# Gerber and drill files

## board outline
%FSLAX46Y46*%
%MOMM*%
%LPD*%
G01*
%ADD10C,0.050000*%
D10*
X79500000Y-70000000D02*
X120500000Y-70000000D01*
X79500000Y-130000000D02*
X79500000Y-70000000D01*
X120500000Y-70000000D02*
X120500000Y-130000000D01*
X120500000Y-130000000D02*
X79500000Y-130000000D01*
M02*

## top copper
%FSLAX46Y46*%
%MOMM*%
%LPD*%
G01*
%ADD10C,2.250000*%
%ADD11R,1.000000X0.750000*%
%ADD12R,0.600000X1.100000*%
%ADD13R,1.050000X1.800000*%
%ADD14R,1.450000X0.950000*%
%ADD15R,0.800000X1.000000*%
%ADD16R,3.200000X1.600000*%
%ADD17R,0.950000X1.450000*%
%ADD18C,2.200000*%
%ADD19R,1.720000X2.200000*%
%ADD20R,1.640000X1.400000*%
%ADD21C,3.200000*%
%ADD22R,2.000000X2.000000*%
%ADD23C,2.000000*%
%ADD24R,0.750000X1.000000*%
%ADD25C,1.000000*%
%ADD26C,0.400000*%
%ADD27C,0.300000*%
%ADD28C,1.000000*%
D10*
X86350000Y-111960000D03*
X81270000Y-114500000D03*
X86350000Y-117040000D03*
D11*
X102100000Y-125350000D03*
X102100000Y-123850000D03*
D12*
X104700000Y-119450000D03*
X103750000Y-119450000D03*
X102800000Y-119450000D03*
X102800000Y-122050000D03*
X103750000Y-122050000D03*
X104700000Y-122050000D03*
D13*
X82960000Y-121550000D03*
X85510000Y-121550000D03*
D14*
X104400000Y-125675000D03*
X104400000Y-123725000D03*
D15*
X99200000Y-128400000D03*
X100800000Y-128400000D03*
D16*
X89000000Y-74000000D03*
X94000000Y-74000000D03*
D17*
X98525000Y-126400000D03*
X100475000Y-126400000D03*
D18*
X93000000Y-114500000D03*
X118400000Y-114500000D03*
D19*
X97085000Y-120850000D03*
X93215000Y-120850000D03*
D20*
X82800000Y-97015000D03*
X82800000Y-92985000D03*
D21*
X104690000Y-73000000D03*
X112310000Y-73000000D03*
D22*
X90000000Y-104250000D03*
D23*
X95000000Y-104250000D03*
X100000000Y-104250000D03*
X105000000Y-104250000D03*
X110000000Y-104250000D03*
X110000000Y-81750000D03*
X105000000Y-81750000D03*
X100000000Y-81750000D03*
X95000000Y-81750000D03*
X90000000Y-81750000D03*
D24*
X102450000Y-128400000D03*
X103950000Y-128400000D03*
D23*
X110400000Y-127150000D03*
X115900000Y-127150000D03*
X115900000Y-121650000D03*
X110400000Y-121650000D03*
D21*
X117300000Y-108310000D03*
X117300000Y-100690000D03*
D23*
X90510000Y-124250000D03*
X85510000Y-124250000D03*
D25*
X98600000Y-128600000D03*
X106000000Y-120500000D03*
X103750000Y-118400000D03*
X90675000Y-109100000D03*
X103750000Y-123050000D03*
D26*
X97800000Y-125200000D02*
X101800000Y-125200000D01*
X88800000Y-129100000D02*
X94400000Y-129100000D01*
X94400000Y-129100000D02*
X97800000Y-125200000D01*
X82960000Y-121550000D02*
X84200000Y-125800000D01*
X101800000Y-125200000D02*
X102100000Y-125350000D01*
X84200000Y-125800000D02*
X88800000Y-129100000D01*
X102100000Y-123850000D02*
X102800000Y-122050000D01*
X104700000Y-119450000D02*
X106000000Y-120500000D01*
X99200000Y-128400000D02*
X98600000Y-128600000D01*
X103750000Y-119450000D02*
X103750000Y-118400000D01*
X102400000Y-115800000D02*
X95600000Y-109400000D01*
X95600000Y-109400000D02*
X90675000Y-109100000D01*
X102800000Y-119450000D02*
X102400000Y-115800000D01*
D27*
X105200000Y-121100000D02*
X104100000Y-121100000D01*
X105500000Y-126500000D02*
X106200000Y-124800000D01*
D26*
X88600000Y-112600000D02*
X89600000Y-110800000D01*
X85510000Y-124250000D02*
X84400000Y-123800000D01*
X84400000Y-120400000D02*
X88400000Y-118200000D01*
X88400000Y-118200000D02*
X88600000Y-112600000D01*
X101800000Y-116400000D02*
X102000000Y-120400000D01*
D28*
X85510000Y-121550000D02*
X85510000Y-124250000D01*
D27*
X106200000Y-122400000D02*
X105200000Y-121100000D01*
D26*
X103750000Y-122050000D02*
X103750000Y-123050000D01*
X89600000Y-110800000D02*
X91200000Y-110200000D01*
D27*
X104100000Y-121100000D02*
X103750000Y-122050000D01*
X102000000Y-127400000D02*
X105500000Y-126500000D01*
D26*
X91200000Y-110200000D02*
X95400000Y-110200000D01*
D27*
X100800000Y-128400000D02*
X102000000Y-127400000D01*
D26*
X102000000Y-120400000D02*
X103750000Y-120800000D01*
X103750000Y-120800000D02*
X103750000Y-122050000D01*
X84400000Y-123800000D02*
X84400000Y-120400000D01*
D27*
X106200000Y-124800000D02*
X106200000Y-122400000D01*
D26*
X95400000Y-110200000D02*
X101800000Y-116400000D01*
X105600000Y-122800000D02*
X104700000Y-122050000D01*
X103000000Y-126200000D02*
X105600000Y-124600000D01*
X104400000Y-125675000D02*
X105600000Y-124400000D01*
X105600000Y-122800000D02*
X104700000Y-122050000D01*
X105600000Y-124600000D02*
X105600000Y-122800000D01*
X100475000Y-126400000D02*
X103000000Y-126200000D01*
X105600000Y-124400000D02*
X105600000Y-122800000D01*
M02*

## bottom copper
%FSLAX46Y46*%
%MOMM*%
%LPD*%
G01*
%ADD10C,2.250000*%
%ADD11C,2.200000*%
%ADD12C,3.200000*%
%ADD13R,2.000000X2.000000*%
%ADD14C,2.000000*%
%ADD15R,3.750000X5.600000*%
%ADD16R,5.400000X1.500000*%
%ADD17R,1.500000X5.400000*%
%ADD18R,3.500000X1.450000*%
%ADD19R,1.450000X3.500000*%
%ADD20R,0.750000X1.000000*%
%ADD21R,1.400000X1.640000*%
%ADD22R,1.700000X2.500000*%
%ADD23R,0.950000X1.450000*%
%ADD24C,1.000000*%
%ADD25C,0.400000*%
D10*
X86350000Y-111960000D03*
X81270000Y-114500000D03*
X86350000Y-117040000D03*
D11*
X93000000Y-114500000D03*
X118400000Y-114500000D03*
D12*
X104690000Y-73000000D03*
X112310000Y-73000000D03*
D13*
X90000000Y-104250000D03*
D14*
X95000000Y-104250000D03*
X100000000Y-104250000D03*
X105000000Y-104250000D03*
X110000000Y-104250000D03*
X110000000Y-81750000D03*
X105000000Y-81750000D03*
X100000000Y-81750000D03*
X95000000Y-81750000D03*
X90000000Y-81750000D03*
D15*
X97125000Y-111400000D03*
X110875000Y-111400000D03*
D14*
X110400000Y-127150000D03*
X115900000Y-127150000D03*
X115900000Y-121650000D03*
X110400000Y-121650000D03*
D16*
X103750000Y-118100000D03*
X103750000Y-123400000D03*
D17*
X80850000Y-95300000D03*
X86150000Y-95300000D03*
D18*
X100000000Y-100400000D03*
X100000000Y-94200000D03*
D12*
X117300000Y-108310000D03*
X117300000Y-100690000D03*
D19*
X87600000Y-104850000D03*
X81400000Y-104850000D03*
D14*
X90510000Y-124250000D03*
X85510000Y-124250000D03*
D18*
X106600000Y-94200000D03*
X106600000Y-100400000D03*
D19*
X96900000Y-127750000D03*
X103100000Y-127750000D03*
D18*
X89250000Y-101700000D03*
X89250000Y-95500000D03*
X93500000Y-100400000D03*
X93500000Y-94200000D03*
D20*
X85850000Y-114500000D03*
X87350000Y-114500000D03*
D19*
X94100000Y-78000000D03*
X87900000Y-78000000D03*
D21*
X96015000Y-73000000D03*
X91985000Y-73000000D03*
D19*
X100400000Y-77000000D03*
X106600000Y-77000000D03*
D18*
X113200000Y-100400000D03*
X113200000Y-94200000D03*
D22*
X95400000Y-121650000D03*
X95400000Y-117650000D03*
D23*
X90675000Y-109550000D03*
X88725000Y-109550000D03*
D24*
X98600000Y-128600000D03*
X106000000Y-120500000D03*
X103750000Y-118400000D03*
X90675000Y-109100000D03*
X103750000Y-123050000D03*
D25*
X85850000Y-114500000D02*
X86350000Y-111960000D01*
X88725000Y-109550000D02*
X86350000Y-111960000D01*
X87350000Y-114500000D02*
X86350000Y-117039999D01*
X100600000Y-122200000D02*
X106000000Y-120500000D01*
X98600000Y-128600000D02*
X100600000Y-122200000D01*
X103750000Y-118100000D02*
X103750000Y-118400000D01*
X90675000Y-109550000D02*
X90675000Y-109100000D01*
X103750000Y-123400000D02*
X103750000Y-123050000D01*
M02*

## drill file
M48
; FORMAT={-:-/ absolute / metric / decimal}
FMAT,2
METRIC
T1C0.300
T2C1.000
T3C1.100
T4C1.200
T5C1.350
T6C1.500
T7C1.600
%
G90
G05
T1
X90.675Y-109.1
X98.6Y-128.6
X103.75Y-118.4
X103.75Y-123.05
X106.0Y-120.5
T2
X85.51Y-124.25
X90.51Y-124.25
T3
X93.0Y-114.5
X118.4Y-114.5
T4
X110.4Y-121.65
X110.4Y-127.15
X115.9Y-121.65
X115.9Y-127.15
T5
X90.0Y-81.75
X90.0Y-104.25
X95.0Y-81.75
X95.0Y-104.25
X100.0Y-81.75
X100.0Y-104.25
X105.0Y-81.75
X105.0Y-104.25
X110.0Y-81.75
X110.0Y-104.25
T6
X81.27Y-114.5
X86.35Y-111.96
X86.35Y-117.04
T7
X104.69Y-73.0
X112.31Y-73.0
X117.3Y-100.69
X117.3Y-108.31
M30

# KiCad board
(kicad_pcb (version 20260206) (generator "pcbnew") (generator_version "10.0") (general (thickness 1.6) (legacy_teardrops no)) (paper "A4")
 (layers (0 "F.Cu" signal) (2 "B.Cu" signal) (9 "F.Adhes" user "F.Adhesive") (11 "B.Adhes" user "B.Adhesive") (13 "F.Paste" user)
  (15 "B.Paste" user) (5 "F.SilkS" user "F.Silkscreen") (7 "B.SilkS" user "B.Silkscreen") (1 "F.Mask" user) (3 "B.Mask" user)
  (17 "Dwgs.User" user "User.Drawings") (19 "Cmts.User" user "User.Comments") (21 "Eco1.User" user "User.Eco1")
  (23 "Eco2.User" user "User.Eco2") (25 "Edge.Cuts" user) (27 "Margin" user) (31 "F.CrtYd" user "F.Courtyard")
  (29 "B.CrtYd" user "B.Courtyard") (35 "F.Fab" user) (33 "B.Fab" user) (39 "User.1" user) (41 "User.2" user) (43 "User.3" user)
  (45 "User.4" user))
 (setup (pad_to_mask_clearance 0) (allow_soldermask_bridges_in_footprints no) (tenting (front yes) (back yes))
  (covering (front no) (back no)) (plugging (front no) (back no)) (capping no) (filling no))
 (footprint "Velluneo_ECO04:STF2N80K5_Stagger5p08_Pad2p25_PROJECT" (layer "F.Cu") (at 86.35 114.5 -90)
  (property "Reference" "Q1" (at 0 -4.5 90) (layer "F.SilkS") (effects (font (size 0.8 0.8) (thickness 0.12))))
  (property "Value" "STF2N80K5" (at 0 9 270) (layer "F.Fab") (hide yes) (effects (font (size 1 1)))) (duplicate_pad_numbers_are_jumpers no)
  (pad "1" thru_hole circle (at -2.54 0 270) (size 2.25 2.25) (drill 1.5) (layers "*.Cu" "*.Mask") (remove_unused_layers no) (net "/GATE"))
  (pad "2" thru_hole circle (at 0 5.08 270) (size 2.25 2.25) (drill 1.5) (layers "*.Cu" "*.Mask") (remove_unused_layers no) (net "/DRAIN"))
  (pad "3" thru_hole circle (at 2.54 0 270) (size 2.25 2.25) (drill 1.5) (layers "*.Cu" "*.Mask") (remove_unused_layers no) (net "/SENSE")))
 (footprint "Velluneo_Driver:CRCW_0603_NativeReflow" (layer "F.Cu") (at 102.1 124.6 90)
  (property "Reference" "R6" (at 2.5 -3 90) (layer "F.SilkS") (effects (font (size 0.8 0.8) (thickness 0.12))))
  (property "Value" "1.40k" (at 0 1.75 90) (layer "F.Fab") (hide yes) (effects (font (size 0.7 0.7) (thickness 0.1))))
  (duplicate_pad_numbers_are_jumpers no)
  (pad "1" smd rect (at -0.75 0 90) (size 0.75 1) (layers "F.Cu" "F.Mask" "F.Paste") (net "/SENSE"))
  (pad "2" smd rect (at 0.75 0 90) (size 0.75 1) (layers "F.Cu" "F.Mask" "F.Paste") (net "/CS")))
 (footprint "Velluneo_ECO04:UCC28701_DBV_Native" (layer "F.Cu") (at 103.75 120.75 -90)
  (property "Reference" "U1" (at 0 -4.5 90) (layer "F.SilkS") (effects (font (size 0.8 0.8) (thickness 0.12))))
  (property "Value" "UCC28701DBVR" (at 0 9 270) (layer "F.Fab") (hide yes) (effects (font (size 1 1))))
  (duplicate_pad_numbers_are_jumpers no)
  (pad "1" smd rect (at -1.3 -0.95 270) (size 1.1 0.6) (layers "F.Cu" "F.Mask" "F.Paste") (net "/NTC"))
  (pad "2" smd rect (at -1.3 0 270) (size 1.1 0.6) (layers "F.Cu" "F.Mask" "F.Paste") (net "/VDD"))
  (pad "3" smd rect (at -1.3 0.95 270) (size 1.1 0.6) (layers "F.Cu" "F.Mask" "F.Paste") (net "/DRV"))
  (pad "4" smd rect (at 1.3 0.95 270) (size 1.1 0.6) (layers "F.Cu" "F.Mask" "F.Paste") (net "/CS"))
  (pad "5" smd rect (at 1.3 0 270) (size 1.1 0.6) (layers "F.Cu" "F.Mask" "F.Paste") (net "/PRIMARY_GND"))
  (pad "6" smd rect (at 1.3 -0.95 270) (size 1.1 0.6) (layers "F.Cu" "F.Mask" "F.Paste") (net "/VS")))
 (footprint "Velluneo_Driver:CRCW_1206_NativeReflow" (layer "F.Cu") (at 84.235 121.55)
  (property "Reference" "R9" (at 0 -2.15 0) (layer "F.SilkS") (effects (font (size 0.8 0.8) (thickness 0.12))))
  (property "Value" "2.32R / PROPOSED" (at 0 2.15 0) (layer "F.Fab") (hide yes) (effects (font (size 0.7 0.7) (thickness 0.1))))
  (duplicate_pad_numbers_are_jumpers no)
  (pad "1" smd rect (at -1.275 0) (size 1.05 1.8) (layers "F.Cu" "F.Mask" "F.Paste") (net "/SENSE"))
  (pad "2" smd rect (at 1.275 0) (size 1.05 1.8) (layers "F.Cu" "F.Mask" "F.Paste") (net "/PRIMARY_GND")))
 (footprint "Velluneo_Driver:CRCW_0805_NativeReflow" (layer "F.Cu") (at 104.4 124.7 90)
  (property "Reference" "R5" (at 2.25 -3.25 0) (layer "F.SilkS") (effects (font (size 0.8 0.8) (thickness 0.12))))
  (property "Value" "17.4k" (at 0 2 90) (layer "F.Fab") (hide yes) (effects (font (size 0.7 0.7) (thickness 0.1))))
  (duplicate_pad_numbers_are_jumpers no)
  (pad "1" smd rect (at -0.975 0 90) (size 0.95 1.45) (layers "F.Cu" "F.Mask" "F.Paste") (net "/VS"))
  (pad "2" smd rect (at 0.975 0 90) (size 0.95 1.45) (layers "F.Cu" "F.Mask" "F.Paste") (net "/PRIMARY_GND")))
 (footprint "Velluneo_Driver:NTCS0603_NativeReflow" (layer "F.Cu") (at 100 128.4)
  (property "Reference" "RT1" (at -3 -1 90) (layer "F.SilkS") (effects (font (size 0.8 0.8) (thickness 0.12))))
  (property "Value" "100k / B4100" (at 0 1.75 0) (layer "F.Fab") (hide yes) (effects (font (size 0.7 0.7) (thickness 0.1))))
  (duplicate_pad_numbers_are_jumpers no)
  (pad "1" smd rect (at -0.8 0) (size 0.8 1) (layers "F.Cu" "F.Mask" "F.Paste") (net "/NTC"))
  (pad "2" smd rect (at 0.8 0) (size 0.8 1) (layers "F.Cu" "F.Mask" "F.Paste") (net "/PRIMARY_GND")))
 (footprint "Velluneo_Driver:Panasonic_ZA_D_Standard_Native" (layer "F.Cu") (at 91.5 74)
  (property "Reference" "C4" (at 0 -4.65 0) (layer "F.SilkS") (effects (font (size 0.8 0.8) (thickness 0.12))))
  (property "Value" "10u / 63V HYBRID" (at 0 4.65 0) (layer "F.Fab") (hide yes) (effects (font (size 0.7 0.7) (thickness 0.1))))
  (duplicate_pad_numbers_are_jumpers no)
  (pad "1" smd rect (at -2.5 0) (size 3.2 1.6) (layers "F.Cu" "F.Mask" "F.Paste") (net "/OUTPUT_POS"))
  (pad "2" smd rect (at 2.5 0) (size 3.2 1.6) (layers "F.Cu" "F.Mask" "F.Paste") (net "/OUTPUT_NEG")))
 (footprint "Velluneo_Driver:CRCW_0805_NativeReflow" (layer "F.Cu") (at 99.5 126.4)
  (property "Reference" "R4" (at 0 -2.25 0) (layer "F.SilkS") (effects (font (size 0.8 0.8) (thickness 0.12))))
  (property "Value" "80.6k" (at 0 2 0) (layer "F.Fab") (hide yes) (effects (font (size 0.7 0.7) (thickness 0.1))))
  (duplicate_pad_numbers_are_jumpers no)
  (pad "1" smd rect (at -0.975 0) (size 0.95 1.45) (layers "F.Cu" "F.Mask" "F.Paste") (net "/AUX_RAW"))
  (pad "2" smd rect (at 0.975 0) (size 0.95 1.45) (layers "F.Cu" "F.Mask" "F.Paste") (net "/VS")))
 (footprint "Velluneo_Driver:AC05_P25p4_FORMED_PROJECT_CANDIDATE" (layer "F.Cu") (at 105.7 114.5)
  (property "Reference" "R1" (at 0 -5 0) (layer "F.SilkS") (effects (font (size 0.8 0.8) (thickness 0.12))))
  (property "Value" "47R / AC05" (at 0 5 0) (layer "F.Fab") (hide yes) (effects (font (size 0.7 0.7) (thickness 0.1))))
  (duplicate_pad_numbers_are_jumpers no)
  (pad "1" thru_hole circle (at -12.7 0) (size 2.2 2.2) (drill 1.1) (layers "*.Cu" "*.Mask") (remove_unused_layers no) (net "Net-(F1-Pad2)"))
  (pad "2" thru_hole circle (at 12.7 0) (size 2.2 2.2) (drill 1.1) (layers "*.Cu" "*.Mask") (remove_unused_layers no)
   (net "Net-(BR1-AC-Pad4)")))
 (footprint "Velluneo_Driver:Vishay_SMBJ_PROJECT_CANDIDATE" (layer "F.Cu") (at 95.15 120.85 180)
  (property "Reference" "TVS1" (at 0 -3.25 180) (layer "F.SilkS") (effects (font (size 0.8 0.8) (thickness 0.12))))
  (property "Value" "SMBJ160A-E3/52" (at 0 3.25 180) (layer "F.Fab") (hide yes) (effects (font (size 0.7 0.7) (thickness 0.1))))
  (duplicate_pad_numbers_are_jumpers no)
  (pad "1" smd rect (at -1.935 0 180) (size 1.72 2.2) (layers "F.Cu" "F.Mask" "F.Paste") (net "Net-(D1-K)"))
  (pad "2" smd rect (at 1.935 0 180) (size 1.72 2.2) (layers "F.Cu" "F.Mask" "F.Paste") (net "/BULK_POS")))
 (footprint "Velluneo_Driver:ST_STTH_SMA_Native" (layer "F.Cu") (at 82.8 95 90)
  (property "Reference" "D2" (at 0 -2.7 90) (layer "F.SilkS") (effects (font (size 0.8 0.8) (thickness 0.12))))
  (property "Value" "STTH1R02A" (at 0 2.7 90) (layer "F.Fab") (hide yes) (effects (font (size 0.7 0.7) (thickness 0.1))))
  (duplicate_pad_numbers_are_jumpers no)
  (pad "1" smd rect (at -2.015 0 90) (size 1.4 1.64) (layers "F.Cu" "F.Mask" "F.Paste") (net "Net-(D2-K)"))
  (pad "2" smd rect (at 2.015 0 90) (size 1.4 1.64) (layers "F.Cu" "F.Mask" "F.Paste") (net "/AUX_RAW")))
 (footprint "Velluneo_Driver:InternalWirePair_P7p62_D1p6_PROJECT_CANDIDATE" (layer "F.Cu") (at 108.5 73)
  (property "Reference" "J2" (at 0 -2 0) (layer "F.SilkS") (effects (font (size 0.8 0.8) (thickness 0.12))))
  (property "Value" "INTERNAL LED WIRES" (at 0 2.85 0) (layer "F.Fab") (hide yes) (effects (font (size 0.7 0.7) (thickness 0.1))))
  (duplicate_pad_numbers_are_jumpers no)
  (pad "1" thru_hole circle (at -3.81 0) (size 3.2 3.2) (drill 1.6) (layers "*.Cu" "*.Mask") (remove_unused_layers no) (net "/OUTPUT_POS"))
  (pad "2" thru_hole circle (at 3.81 0) (size 3.2 3.2) (drill 1.6) (layers "*.Cu" "*.Mask") (remove_unused_layers no) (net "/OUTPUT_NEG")))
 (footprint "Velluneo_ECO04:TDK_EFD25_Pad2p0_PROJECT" (layer "F.Cu") (at 100 93)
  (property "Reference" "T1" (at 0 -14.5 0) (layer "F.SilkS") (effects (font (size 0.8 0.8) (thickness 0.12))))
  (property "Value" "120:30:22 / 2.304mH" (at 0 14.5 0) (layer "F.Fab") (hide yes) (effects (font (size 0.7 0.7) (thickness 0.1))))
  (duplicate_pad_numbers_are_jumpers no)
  (pad "1" thru_hole rect (at -10 11.25) (size 2 2) (drill 1.35) (layers "*.Cu" "*.Mask") (remove_unused_layers no) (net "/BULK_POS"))
  (pad "2" thru_hole circle (at -5 11.25) (size 2 2) (drill 1.35) (layers "*.Cu" "*.Mask") (remove_unused_layers no) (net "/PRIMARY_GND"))
  (pad "3" thru_hole circle (at 0 11.25) (size 2 2) (drill 1.35) (layers "*.Cu" "*.Mask") (remove_unused_layers no)
   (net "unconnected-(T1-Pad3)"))
  (pad "4" thru_hole circle (at 5 11.25) (size 2 2) (drill 1.35) (layers "*.Cu" "*.Mask") (remove_unused_layers no) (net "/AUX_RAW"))
  (pad "5" thru_hole circle (at 10 11.25) (size 2 2) (drill 1.35) (layers "*.Cu" "*.Mask") (remove_unused_layers no) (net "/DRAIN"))
  (pad "6" thru_hole circle (at 10 -11.25) (size 2 2) (drill 1.35) (layers "*.Cu" "*.Mask") (remove_unused_layers no) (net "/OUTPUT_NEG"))
  (pad "7" thru_hole circle (at 5 -11.25) (size 2 2) (drill 1.35) (layers "*.Cu" "*.Mask") (remove_unused_layers no)
   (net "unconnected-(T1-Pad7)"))
  (pad "8" thru_hole circle (at 0 -11.25) (size 2 2) (drill 1.35) (layers "*.Cu" "*.Mask") (remove_unused_layers no)
   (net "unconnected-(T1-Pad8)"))
  (pad "9" thru_hole circle (at -5 -11.25) (size 2 2) (drill 1.35) (layers "*.Cu" "*.Mask") (remove_unused_layers no)
   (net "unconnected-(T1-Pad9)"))
  (pad "10" thru_hole circle (at -10 -11.25) (size 2 2) (drill 1.35) (layers "*.Cu" "*.Mask") (remove_unused_layers no)
   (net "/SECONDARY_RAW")))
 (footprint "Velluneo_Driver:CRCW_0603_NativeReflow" (layer "F.Cu") (at 103.2 128.4)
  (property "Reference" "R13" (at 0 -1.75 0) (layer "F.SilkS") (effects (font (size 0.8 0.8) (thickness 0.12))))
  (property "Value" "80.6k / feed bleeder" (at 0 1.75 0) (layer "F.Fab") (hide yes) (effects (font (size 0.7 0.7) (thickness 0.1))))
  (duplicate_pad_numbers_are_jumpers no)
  (pad "1" smd rect (at -0.75 0) (size 0.75 1) (layers "F.Cu" "F.Mask" "F.Paste") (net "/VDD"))
  (pad "2" smd rect (at 0.75 0) (size 0.75 1) (layers "F.Cu" "F.Mask" "F.Paste") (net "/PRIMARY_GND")))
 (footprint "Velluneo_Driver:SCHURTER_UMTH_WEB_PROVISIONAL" (layer "B.Cu") (at 104 111.4)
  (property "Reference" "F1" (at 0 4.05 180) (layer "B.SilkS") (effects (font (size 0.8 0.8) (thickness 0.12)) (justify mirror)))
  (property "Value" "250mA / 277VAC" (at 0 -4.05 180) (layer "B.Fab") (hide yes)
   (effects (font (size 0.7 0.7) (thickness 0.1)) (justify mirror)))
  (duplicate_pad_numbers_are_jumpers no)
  (pad "1" smd rect (at -6.875 0) (size 3.75 5.6) (layers "B.Cu" "B.Mask" "B.Paste") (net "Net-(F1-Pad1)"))
  (pad "2" smd rect (at 6.875 0) (size 3.75 5.6) (layers "B.Cu" "B.Mask" "B.Paste") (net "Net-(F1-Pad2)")))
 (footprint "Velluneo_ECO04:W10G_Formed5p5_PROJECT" (layer "B.Cu") (at 113.15 124.4)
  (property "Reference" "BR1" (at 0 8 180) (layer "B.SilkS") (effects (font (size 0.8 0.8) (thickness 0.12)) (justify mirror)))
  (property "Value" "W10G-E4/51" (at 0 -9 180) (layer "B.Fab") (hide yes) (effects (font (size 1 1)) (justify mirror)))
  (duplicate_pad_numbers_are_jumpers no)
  (pad "1" thru_hole circle (at -2.75 2.75) (size 2 2) (drill 1.2) (layers "*.Cu" "*.Mask") (remove_unused_layers no) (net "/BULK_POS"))
  (pad "2" thru_hole circle (at 2.75 2.75) (size 2 2) (drill 1.2) (layers "*.Cu" "*.Mask") (remove_unused_layers no)
   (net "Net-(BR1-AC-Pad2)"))
  (pad "3" thru_hole circle (at 2.75 -2.75) (size 2 2) (drill 1.2) (layers "*.Cu" "*.Mask") (remove_unused_layers no) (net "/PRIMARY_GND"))
  (pad "4" thru_hole circle (at -2.75 -2.75) (size 2 2) (drill 1.2) (layers "*.Cu" "*.Mask") (remove_unused_layers no)
   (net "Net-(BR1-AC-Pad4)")))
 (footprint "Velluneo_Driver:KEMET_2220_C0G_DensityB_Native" (layer "B.Cu") (at 103.75 120.75 -90)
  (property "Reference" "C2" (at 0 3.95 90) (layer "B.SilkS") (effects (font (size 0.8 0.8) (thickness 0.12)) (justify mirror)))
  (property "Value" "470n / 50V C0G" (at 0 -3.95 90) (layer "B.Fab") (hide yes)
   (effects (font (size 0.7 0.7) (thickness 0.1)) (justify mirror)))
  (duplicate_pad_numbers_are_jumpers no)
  (pad "1" smd rect (at -2.65 0 270) (size 1.5 5.4) (layers "B.Cu" "B.Mask" "B.Paste") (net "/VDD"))
  (pad "2" smd rect (at 2.65 0 270) (size 1.5 5.4) (layers "B.Cu" "B.Mask" "B.Paste") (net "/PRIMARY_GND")))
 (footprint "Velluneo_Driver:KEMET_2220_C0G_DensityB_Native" (layer "B.Cu") (at 83.5 95.3)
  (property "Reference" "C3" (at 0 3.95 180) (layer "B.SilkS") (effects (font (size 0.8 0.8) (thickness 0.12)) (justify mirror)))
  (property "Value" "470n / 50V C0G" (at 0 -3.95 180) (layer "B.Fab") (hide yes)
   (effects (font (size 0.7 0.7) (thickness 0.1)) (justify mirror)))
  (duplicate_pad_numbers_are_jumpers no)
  (pad "1" smd rect (at -2.65 0) (size 1.5 5.4) (layers "B.Cu" "B.Mask" "B.Paste") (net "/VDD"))
  (pad "2" smd rect (at 2.65 0) (size 1.5 5.4) (layers "B.Cu" "B.Mask" "B.Paste") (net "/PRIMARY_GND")))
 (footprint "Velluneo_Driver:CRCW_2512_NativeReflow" (layer "B.Cu") (at 100 97.3 90)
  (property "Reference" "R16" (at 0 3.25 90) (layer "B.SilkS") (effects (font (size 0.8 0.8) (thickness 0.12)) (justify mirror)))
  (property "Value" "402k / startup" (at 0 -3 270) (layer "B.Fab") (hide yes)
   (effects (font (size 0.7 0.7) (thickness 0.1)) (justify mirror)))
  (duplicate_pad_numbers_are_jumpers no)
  (pad "1" smd rect (at -3.1 0 90) (size 1.45 3.5) (layers "B.Cu" "B.Mask" "B.Paste") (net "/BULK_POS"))
  (pad "2" smd rect (at 3.1 0 90) (size 1.45 3.5) (layers "B.Cu" "B.Mask" "B.Paste") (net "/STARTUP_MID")))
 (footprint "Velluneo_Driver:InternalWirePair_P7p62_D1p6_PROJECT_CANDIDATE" (layer "B.Cu") (at 117.3 104.5 90)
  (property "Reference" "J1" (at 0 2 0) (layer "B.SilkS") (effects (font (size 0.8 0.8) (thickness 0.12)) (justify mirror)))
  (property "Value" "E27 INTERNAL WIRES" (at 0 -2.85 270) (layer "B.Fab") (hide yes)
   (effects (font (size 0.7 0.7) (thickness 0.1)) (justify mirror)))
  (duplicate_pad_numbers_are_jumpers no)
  (pad "1" thru_hole circle (at -3.81 0 90) (size 3.2 3.2) (drill 1.6) (layers "*.Cu" "*.Mask") (remove_unused_layers no)
   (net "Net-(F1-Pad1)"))
  (pad "2" thru_hole circle (at 3.81 0 90) (size 3.2 3.2) (drill 1.6) (layers "*.Cu" "*.Mask") (remove_unused_layers no)
   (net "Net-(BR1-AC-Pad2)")))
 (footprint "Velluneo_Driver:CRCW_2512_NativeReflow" (layer "B.Cu") (at 84.5 104.85 180)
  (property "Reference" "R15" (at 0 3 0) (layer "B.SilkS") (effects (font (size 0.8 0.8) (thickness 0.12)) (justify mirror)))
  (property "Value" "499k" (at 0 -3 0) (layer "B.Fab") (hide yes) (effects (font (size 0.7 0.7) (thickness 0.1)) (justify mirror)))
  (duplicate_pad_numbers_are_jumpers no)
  (pad "1" smd rect (at -3.1 0 180) (size 1.45 3.5) (layers "B.Cu" "B.Mask" "B.Paste") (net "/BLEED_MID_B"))
  (pad "2" smd rect (at 3.1 0 180) (size 1.45 3.5) (layers "B.Cu" "B.Mask" "B.Paste") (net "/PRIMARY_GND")))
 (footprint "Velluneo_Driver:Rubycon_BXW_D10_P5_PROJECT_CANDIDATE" (layer "B.Cu") (at 88.01 124.25 180)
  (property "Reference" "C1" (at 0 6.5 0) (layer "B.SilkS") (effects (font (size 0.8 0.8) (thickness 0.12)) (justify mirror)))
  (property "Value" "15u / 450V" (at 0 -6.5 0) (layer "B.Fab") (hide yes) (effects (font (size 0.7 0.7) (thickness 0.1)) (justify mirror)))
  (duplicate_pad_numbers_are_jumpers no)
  (pad "1" thru_hole circle (at -2.5 0 180) (size 2 2) (drill 1) (layers "*.Cu" "*.Mask") (remove_unused_layers no) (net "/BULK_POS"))
  (pad "2" thru_hole circle (at 2.5 0 180) (size 2 2) (drill 1) (layers "*.Cu" "*.Mask") (remove_unused_layers no) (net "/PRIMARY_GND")))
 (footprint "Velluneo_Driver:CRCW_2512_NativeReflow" (layer "B.Cu") (at 106.6 97.3 -90)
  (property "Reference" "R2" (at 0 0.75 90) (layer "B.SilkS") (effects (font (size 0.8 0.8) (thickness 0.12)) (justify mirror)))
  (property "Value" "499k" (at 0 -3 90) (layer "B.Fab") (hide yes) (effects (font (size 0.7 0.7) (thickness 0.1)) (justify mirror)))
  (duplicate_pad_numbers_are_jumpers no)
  (pad "1" smd rect (at -3.1 0 270) (size 1.45 3.5) (layers "B.Cu" "B.Mask" "B.Paste") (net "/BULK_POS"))
  (pad "2" smd rect (at 3.1 0 270) (size 1.45 3.5) (layers "B.Cu" "B.Mask" "B.Paste") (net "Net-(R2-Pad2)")))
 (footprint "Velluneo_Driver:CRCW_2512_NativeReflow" (layer "B.Cu") (at 100 127.75)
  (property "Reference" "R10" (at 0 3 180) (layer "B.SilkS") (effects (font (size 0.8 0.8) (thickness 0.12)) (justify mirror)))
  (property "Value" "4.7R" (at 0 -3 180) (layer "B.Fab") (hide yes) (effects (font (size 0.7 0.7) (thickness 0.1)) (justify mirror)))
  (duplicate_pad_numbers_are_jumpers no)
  (pad "1" smd rect (at -3.1 0) (size 1.45 3.5) (layers "B.Cu" "B.Mask" "B.Paste") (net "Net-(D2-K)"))
  (pad "2" smd rect (at 3.1 0) (size 1.45 3.5) (layers "B.Cu" "B.Mask" "B.Paste") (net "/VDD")))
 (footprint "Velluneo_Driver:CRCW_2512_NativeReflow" (layer "B.Cu") (at 89.25 98.6 90)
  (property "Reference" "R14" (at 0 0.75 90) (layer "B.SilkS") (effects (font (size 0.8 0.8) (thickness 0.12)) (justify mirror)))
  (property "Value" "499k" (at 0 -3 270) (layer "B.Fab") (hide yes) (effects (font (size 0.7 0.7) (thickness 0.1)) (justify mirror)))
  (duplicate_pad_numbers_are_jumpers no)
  (pad "1" smd rect (at -3.1 0 90) (size 1.45 3.5) (layers "B.Cu" "B.Mask" "B.Paste") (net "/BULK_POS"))
  (pad "2" smd rect (at 3.1 0 90) (size 1.45 3.5) (layers "B.Cu" "B.Mask" "B.Paste") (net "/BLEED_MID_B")))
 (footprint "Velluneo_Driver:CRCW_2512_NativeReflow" (layer "B.Cu") (at 93.5 97.3 90)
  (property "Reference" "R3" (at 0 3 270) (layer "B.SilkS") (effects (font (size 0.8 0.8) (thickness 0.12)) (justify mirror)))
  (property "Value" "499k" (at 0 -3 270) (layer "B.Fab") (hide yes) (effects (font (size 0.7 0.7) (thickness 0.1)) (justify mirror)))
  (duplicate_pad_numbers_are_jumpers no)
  (pad "1" smd rect (at -3.1 0 90) (size 1.45 3.5) (layers "B.Cu" "B.Mask" "B.Paste") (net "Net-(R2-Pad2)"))
  (pad "2" smd rect (at 3.1 0 90) (size 1.45 3.5) (layers "B.Cu" "B.Mask" "B.Paste") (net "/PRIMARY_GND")))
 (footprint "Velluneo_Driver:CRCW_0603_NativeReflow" (layer "B.Cu") (at 86.6 114.5)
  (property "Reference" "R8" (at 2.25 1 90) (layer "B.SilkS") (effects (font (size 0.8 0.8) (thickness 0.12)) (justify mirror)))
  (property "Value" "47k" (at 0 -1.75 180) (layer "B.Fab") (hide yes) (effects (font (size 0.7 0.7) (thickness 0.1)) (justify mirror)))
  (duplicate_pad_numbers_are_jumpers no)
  (pad "1" smd rect (at -0.75 0) (size 0.75 1) (layers "B.Cu" "B.Mask" "B.Paste") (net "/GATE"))
  (pad "2" smd rect (at 0.75 0) (size 0.75 1) (layers "B.Cu" "B.Mask" "B.Paste") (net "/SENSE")))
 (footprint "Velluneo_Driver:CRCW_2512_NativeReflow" (layer "B.Cu") (at 91 78 180)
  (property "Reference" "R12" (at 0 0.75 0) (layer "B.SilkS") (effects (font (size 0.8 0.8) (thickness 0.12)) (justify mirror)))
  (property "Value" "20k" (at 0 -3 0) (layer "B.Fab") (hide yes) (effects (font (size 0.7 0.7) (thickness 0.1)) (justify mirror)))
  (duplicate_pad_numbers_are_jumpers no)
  (pad "1" smd rect (at -3.1 0 180) (size 1.45 3.5) (layers "B.Cu" "B.Mask" "B.Paste") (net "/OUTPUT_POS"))
  (pad "2" smd rect (at 3.1 0 180) (size 1.45 3.5) (layers "B.Cu" "B.Mask" "B.Paste") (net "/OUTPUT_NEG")))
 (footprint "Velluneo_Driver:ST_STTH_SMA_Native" (layer "B.Cu") (at 94 73 180)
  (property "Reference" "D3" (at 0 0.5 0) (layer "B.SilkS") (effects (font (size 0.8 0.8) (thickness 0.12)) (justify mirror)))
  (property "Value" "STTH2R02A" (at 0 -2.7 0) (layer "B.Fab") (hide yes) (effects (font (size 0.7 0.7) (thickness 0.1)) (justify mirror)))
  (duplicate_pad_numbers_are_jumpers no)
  (pad "1" smd rect (at -2.015 0 180) (size 1.4 1.64) (layers "B.Cu" "B.Mask" "B.Paste") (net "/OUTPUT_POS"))
  (pad "2" smd rect (at 2.015 0 180) (size 1.4 1.64) (layers "B.Cu" "B.Mask" "B.Paste") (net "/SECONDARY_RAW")))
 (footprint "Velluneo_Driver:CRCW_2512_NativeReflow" (layer "B.Cu") (at 103.5 77)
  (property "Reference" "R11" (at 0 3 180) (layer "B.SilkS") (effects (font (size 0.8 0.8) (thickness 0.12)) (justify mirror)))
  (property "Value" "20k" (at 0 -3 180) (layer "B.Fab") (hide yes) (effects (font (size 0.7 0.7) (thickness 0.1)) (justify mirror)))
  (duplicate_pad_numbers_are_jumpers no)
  (pad "1" smd rect (at -3.1 0) (size 1.45 3.5) (layers "B.Cu" "B.Mask" "B.Paste") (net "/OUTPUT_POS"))
  (pad "2" smd rect (at 3.1 0) (size 1.45 3.5) (layers "B.Cu" "B.Mask" "B.Paste") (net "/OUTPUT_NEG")))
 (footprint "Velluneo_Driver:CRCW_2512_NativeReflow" (layer "B.Cu") (at 113.2 97.3 90)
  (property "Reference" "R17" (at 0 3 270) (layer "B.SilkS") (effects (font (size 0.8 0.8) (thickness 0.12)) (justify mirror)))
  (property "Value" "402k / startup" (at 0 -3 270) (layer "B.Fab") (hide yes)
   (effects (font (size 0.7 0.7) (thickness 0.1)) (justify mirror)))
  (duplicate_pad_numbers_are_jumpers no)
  (pad "1" smd rect (at -3.1 0 90) (size 1.45 3.5) (layers "B.Cu" "B.Mask" "B.Paste") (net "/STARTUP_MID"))
  (pad "2" smd rect (at 3.1 0 90) (size 1.45 3.5) (layers "B.Cu" "B.Mask" "B.Paste") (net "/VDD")))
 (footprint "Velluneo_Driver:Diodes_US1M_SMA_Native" (layer "B.Cu") (at 95.4 119.65 90)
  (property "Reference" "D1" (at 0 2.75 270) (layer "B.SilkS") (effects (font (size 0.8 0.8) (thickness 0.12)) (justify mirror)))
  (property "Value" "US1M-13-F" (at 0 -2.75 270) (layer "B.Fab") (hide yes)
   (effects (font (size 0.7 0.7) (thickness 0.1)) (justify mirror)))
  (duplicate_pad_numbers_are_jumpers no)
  (pad "1" smd rect (at -2 0 90) (size 2.5 1.7) (layers "B.Cu" "B.Mask" "B.Paste") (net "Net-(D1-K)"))
  (pad "2" smd rect (at 2 0 90) (size 2.5 1.7) (layers "B.Cu" "B.Mask" "B.Paste") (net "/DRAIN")))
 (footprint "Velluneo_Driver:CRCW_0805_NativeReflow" (layer "B.Cu") (at 89.7 109.55 180)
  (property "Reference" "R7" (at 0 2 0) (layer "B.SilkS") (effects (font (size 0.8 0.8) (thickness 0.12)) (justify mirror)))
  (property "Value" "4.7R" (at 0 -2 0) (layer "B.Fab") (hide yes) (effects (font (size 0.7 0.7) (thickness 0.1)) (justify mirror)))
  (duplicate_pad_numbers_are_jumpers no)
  (pad "1" smd rect (at -0.975 0 180) (size 0.95 1.45) (layers "B.Cu" "B.Mask" "B.Paste") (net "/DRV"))
  (pad "2" smd rect (at 0.975 0 180) (size 0.95 1.45) (layers "B.Cu" "B.Mask" "B.Paste") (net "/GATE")))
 (gr_line (start 79.5 70) (end 120.5 70) (stroke (width 0.05) (type default)) (layer "Edge.Cuts"))
 (gr_line (start 79.5 130) (end 79.5 70) (stroke (width 0.05) (type default)) (layer "Edge.Cuts"))
 (gr_line (start 120.5 70) (end 120.5 130) (stroke (width 0.05) (type default)) (layer "Edge.Cuts"))
 (gr_line (start 120.5 130) (end 79.5 130) (stroke (width 0.05) (type default)) (layer "Edge.Cuts"))
 (segment (start 85.85 114.5) (end 86.35 111.96) (width 0.4) (layer "B.Cu") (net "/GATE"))
 (segment (start 88.725 109.55) (end 86.35 111.96) (width 0.4) (layer "B.Cu") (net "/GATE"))
 (segment (start 97.8 125.2) (end 101.8 125.2) (width 0.4) (layer "F.Cu") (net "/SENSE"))
 (segment (start 88.8 129.1) (end 94.4 129.1) (width 0.4) (layer "F.Cu") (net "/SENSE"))
 (segment (start 94.4 129.1) (end 97.8 125.2) (width 0.4) (layer "F.Cu") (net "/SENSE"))
 (segment (start 82.96 121.55) (end 84.2 125.8) (width 0.4) (layer "F.Cu") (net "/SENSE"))
 (segment (start 101.8 125.2) (end 102.1 125.35) (width 0.4) (layer "F.Cu") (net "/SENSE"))
 (segment (start 84.2 125.8) (end 88.8 129.1) (width 0.4) (layer "F.Cu") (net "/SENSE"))
 (segment (start 87.35 114.5) (end 86.35 117.039999) (width 0.4) (layer "B.Cu") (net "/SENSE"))
 (segment (start 102.1 123.85) (end 102.8 122.05) (width 0.4) (layer "F.Cu") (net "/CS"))
 (segment (start 104.7 119.45) (end 106 120.5) (width 0.4) (layer "F.Cu") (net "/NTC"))
 (segment (start 99.2 128.4) (end 98.6 128.6) (width 0.4) (layer "F.Cu") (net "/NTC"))
 (via (at 98.6 128.6) (size 1) (drill 0.3) (layers "F.Cu" "B.Cu") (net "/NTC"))
 (via (at 106 120.5) (size 1) (drill 0.3) (layers "F.Cu" "B.Cu") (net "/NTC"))
 (segment (start 100.6 122.2) (end 106 120.5) (width 0.4) (layer "B.Cu") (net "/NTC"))
 (segment (start 98.6 128.6) (end 100.6 122.2) (width 0.4) (layer "B.Cu") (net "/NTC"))
 (segment (start 103.75 119.45) (end 103.75 118.4) (width 0.4) (layer "F.Cu") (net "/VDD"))
 (via (at 103.75 118.4) (size 1) (drill 0.3) (layers "F.Cu" "B.Cu") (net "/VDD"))
 (segment (start 103.75 118.1) (end 103.75 118.4) (width 0.4) (layer "B.Cu") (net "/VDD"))
 (segment (start 102.4 115.8) (end 95.6 109.4) (width 0.4) (layer "F.Cu") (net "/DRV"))
 (segment (start 95.6 109.4) (end 90.675 109.1) (width 0.4) (layer "F.Cu") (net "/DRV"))
 (segment (start 102.8 119.45) (end 102.4 115.8) (width 0.4) (layer "F.Cu") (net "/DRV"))
 (via (at 90.675 109.1) (size 1) (drill 0.3) (layers "F.Cu" "B.Cu") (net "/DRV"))
 (segment (start 90.675 109.55) (end 90.675 109.1) (width 0.4) (layer "B.Cu") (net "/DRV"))
 (segment (start 105.2 121.1) (end 104.1 121.1) (width 0.3) (layer "F.Cu") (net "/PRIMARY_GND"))
 (segment (start 105.5 126.5) (end 106.2 124.8) (width 0.3) (layer "F.Cu") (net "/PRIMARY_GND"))
 (segment (start 88.6 112.6) (end 89.6 110.8) (width 0.4) (layer "F.Cu") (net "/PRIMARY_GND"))
 (segment (start 85.51 124.25) (end 84.4 123.8) (width 0.4) (layer "F.Cu") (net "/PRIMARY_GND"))
 (segment (start 84.4 120.4) (end 88.4 118.2) (width 0.4) (layer "F.Cu") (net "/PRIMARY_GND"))
 (segment (start 88.4 118.2) (end 88.6 112.6) (width 0.4) (layer "F.Cu") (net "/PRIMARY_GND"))
 (segment (start 101.8 116.4) (end 102 120.4) (width 0.4) (layer "F.Cu") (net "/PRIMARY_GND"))
 (segment (start 85.51 121.55) (end 85.51 124.25) (width 1) (layer "F.Cu") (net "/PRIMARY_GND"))
 (segment (start 106.2 122.4) (end 105.2 121.1) (width 0.3) (layer "F.Cu") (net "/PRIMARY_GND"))
 (segment (start 103.75 122.05) (end 103.75 123.05) (width 0.4) (layer "F.Cu") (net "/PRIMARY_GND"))
 (segment (start 89.6 110.8) (end 91.2 110.2) (width 0.4) (layer "F.Cu") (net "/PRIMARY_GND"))
 (segment (start 104.1 121.1) (end 103.75 122.05) (width 0.3) (layer "F.Cu") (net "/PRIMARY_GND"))
 (segment (start 102 127.4) (end 105.5 126.5) (width 0.3) (layer "F.Cu") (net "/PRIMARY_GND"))
 (segment (start 91.2 110.2) (end 95.4 110.2) (width 0.4) (layer "F.Cu") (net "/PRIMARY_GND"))
 (segment (start 100.8 128.4) (end 102 127.4) (width 0.3) (layer "F.Cu") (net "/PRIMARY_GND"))
 (segment (start 102 120.4) (end 103.75 120.8) (width 0.4) (layer "F.Cu") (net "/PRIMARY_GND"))
 (segment (start 103.75 120.8) (end 103.75 122.05) (width 0.4) (layer "F.Cu") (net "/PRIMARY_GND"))
 (segment (start 84.4 123.8) (end 84.4 120.4) (width 0.4) (layer "F.Cu") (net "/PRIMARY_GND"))
 (segment (start 106.2 124.8) (end 106.2 122.4) (width 0.3) (layer "F.Cu") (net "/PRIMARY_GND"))
 (segment (start 95.4 110.2) (end 101.8 116.4) (width 0.4) (layer "F.Cu") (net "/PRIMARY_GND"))
 (via (at 103.75 123.05) (size 1) (drill 0.3) (layers "F.Cu" "B.Cu") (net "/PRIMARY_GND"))
 (segment (start 103.75 123.4) (end 103.75 123.05) (width 0.4) (layer "B.Cu") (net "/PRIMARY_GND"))
 (segment (start 105.6 122.8) (end 104.7 122.05) (width 0.4) (layer "F.Cu") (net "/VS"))
 (segment (start 103 126.2) (end 105.6 124.6) (width 0.4) (layer "F.Cu") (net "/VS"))
 (segment (start 104.4 125.675) (end 105.6 124.4) (width 0.4) (layer "F.Cu") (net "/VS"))
 (segment (start 105.6 122.8) (end 104.7 122.05) (width 0.4) (layer "F.Cu") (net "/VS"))
 (segment (start 105.6 124.6) (end 105.6 122.8) (width 0.4) (layer "F.Cu") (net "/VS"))
 (segment (start 100.475 126.4) (end 103 126.2) (width 0.4) (layer "F.Cu") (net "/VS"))
 (segment (start 105.6 124.4) (end 105.6 122.8) (width 0.4) (layer "F.Cu") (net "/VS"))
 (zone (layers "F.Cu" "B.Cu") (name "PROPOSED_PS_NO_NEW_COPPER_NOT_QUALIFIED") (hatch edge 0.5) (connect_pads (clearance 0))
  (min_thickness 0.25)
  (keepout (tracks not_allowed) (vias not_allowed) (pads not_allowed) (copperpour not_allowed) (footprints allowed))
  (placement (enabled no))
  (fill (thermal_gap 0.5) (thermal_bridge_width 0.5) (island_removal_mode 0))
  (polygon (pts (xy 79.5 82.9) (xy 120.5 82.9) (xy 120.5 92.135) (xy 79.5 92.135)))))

